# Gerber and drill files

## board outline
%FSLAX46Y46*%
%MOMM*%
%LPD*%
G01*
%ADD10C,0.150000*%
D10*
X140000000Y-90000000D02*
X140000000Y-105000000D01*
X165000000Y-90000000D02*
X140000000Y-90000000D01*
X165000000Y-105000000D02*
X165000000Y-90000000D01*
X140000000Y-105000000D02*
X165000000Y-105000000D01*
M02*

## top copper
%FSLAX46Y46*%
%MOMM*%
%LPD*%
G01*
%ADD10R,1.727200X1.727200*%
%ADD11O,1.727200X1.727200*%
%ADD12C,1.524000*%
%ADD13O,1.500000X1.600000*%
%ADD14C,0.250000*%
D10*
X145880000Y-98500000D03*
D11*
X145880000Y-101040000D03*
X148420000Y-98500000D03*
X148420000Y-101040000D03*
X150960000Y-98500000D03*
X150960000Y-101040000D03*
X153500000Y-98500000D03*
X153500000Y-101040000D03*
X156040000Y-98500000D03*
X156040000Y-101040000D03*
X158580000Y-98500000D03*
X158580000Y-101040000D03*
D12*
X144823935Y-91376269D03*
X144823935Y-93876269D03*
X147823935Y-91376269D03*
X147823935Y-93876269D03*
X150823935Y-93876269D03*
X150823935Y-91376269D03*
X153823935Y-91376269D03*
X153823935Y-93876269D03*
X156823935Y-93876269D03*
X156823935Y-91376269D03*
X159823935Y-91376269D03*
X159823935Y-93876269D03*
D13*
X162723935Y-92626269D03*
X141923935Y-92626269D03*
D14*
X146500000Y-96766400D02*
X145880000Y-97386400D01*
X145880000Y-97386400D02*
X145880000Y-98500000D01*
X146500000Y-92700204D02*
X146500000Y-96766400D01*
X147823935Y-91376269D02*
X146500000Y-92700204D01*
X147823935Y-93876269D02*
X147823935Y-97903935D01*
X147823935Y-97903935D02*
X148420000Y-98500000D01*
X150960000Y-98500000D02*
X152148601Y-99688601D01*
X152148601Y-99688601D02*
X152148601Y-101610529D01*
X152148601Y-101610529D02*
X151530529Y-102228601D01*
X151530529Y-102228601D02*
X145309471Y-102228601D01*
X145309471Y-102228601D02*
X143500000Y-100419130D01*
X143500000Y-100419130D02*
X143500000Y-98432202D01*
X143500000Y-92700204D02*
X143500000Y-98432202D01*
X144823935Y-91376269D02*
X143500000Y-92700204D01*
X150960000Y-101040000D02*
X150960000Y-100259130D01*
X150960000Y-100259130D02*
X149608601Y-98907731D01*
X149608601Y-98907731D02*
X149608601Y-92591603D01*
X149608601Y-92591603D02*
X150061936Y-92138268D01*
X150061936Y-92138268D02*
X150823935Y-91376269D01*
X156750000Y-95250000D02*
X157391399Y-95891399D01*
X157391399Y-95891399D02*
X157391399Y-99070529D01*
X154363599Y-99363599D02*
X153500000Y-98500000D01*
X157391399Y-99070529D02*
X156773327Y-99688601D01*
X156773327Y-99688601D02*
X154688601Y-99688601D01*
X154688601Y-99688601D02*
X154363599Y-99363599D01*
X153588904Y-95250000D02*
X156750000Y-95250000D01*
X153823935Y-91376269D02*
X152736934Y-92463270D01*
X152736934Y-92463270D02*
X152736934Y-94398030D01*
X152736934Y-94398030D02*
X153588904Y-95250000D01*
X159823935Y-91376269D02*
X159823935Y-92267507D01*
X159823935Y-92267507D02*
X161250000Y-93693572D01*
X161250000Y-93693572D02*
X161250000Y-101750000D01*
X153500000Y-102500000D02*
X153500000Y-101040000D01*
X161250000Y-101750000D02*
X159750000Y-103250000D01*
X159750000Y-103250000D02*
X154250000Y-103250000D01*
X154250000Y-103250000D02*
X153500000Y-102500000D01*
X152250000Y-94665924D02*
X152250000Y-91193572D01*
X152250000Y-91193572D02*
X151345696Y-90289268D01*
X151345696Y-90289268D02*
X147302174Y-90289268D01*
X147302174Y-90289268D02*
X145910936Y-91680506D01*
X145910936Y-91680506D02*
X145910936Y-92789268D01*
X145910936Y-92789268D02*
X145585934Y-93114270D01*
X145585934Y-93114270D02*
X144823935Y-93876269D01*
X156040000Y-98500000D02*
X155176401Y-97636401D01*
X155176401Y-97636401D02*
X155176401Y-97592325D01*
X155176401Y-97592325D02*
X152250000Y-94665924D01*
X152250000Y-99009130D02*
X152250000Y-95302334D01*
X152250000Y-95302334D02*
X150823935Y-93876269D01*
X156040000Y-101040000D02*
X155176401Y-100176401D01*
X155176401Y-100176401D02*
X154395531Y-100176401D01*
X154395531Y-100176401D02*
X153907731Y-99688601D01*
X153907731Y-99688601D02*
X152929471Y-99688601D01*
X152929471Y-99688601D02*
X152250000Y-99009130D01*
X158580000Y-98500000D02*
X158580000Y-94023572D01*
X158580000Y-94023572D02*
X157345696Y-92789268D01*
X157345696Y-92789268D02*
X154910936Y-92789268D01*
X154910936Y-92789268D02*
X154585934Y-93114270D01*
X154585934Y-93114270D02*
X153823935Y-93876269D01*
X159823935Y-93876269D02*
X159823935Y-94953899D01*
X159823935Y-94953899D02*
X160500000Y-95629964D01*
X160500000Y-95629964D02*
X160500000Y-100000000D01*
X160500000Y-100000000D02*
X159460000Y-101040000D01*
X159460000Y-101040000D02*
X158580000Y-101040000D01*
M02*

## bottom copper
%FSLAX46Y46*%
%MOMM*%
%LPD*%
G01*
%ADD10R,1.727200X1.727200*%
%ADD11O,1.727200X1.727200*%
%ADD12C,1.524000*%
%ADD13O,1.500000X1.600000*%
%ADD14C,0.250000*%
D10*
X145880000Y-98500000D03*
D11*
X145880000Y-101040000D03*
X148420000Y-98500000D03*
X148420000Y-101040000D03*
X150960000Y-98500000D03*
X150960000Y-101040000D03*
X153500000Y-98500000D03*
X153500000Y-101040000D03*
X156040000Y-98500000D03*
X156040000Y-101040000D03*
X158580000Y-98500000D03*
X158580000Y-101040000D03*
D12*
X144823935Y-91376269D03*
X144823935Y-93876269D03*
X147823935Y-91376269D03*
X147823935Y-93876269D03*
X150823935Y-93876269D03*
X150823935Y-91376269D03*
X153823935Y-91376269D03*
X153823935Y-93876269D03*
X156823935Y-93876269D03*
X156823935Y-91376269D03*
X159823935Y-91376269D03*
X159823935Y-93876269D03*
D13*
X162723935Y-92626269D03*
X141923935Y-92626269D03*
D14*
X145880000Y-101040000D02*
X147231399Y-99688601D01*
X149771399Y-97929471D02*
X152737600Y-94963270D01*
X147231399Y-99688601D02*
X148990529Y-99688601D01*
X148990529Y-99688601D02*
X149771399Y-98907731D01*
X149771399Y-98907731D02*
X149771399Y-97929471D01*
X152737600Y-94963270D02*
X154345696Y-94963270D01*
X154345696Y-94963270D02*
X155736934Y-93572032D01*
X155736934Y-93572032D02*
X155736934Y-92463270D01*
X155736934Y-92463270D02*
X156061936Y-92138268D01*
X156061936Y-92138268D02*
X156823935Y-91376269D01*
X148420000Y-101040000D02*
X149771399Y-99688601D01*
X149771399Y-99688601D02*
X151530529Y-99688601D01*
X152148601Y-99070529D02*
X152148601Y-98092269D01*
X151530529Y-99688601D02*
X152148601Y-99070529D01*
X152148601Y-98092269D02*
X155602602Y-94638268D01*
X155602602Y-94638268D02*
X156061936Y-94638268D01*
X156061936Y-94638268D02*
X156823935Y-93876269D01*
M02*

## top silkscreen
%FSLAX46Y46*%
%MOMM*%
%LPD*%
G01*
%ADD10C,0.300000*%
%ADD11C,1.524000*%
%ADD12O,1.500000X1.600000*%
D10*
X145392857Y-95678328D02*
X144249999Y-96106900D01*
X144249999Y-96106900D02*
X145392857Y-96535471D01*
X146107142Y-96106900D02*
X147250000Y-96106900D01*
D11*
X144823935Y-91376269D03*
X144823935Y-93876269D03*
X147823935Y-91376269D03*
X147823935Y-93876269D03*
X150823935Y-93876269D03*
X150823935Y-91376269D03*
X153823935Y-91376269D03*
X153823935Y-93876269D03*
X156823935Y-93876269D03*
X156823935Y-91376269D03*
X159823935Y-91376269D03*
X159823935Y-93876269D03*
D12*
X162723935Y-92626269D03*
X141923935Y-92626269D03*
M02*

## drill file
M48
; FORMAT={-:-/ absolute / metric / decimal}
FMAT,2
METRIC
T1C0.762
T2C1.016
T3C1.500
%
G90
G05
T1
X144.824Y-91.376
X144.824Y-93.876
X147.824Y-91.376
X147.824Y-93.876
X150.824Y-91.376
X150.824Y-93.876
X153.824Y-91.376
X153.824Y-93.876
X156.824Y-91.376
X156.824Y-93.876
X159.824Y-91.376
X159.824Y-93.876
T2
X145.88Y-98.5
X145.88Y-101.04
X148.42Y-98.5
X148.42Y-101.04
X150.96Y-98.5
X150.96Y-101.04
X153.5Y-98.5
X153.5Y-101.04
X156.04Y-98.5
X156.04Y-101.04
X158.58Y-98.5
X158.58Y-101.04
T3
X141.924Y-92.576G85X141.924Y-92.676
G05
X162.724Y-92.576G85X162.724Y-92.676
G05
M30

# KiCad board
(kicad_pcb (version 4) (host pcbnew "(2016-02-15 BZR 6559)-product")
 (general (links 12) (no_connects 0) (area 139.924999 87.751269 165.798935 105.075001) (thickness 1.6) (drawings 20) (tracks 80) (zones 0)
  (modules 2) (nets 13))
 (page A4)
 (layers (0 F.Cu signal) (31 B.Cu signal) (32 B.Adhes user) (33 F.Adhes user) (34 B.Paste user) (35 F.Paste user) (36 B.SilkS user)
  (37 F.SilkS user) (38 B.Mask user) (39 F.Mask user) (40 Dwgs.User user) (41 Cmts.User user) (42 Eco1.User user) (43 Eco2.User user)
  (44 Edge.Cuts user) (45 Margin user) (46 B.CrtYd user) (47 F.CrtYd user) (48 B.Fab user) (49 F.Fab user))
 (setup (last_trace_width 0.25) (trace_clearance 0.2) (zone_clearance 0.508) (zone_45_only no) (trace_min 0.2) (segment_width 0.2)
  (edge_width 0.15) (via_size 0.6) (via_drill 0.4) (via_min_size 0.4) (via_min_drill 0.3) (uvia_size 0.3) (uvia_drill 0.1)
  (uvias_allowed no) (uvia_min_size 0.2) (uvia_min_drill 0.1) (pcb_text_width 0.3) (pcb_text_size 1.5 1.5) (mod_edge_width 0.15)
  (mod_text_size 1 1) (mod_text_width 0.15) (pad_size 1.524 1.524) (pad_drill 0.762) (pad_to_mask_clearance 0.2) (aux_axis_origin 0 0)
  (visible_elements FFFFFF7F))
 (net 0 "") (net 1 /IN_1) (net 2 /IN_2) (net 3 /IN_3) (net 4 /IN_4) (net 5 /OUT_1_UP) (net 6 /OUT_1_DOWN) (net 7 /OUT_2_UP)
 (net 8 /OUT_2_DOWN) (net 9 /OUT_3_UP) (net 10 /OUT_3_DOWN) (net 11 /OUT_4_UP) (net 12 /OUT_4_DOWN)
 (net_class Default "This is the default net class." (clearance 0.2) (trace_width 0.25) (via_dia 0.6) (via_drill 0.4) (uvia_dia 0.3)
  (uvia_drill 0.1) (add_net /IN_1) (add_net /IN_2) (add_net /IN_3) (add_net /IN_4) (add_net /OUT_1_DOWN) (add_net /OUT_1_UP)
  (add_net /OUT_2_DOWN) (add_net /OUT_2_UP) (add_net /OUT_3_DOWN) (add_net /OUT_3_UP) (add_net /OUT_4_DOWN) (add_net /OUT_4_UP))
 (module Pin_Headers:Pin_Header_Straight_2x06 (layer B.Cu) (at 145.88 98.5 270)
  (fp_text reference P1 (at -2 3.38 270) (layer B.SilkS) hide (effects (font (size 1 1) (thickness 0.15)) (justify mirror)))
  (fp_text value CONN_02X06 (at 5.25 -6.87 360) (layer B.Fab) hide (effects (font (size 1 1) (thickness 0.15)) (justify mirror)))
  (pad 1 thru_hole rect (at 0 0 270) (size 1.7272 1.7272) (drill 1.016) (layers *.Cu *.Mask B.SilkS) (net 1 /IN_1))
  (pad 2 thru_hole oval (at 2.54 0 270) (size 1.7272 1.7272) (drill 1.016) (layers *.Cu *.Mask B.SilkS) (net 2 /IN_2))
  (pad 3 thru_hole oval (at 0 -2.54 270) (size 1.7272 1.7272) (drill 1.016) (layers *.Cu *.Mask B.SilkS) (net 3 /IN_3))
  (pad 4 thru_hole oval (at 2.54 -2.54 270) (size 1.7272 1.7272) (drill 1.016) (layers *.Cu *.Mask B.SilkS) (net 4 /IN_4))
  (pad 5 thru_hole oval (at 0 -5.08 270) (size 1.7272 1.7272) (drill 1.016) (layers *.Cu *.Mask B.SilkS) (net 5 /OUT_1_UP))
  (pad 6 thru_hole oval (at 2.54 -5.08 270) (size 1.7272 1.7272) (drill 1.016) (layers *.Cu *.Mask B.SilkS) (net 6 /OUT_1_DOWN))
  (pad 7 thru_hole oval (at 0 -7.62 270) (size 1.7272 1.7272) (drill 1.016) (layers *.Cu *.Mask B.SilkS) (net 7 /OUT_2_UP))
  (pad 8 thru_hole oval (at 2.54 -7.62 270) (size 1.7272 1.7272) (drill 1.016) (layers *.Cu *.Mask B.SilkS) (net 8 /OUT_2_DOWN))
  (pad 9 thru_hole oval (at 0 -10.16 270) (size 1.7272 1.7272) (drill 1.016) (layers *.Cu *.Mask B.SilkS) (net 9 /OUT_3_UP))
  (pad 10 thru_hole oval (at 2.54 -10.16 270) (size 1.7272 1.7272) (drill 1.016) (layers *.Cu *.Mask B.SilkS) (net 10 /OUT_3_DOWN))
  (pad 11 thru_hole oval (at 0 -12.7 270) (size 1.7272 1.7272) (drill 1.016) (layers *.Cu *.Mask B.SilkS) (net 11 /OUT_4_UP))
  (pad 12 thru_hole oval (at 2.54 -12.7 270) (size 1.7272 1.7272) (drill 1.016) (layers *.Cu *.Mask B.SilkS) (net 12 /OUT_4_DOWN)))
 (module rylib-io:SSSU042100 (layer F.Cu) (at 144.823935 91.376269)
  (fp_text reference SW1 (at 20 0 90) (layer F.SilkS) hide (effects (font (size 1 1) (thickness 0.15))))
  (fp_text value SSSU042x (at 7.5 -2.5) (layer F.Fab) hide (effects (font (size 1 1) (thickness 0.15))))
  (pad 5 thru_hole circle (at 0 0) (size 1.524 1.524) (drill 0.762) (layers *.Cu *.Mask F.SilkS) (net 5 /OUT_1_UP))
  (pad 7 thru_hole circle (at 0 2.5) (size 1.524 1.524) (drill 0.762) (layers *.Cu *.Mask F.SilkS) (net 9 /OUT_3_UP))
  (pad 1 thru_hole circle (at 3 0) (size 1.524 1.524) (drill 0.762) (layers *.Cu *.Mask F.SilkS) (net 1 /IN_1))
  (pad 3 thru_hole circle (at 3 2.5) (size 1.524 1.524) (drill 0.762) (layers *.Cu *.Mask F.SilkS) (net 3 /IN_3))
  (pad 11 thru_hole circle (at 6 2.5) (size 1.524 1.524) (drill 0.762) (layers *.Cu *.Mask F.SilkS) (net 10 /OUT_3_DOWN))
  (pad 9 thru_hole circle (at 6 0) (size 1.524 1.524) (drill 0.762) (layers *.Cu *.Mask F.SilkS) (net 6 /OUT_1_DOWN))
  (pad 6 thru_hole circle (at 9 0) (size 1.524 1.524) (drill 0.762) (layers *.Cu *.Mask F.SilkS) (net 7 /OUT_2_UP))
  (pad 8 thru_hole circle (at 9 2.5) (size 1.524 1.524) (drill 0.762) (layers *.Cu *.Mask F.SilkS) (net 11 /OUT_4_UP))
  (pad 4 thru_hole circle (at 12 2.5) (size 1.524 1.524) (drill 0.762) (layers *.Cu *.Mask F.SilkS) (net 4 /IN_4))
  (pad 2 thru_hole circle (at 12 0) (size 1.524 1.524) (drill 0.762) (layers *.Cu *.Mask F.SilkS) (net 2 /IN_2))
  (pad 10 thru_hole circle (at 15 0) (size 1.524 1.524) (drill 0.762) (layers *.Cu *.Mask F.SilkS) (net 8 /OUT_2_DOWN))
  (pad 12 thru_hole circle (at 15 2.5) (size 1.524 1.524) (drill 0.762) (layers *.Cu *.Mask F.SilkS) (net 12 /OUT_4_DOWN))
  (pad "" thru_hole oval (at 17.9 1.25) (size 1.5 1.6) (drill oval 1.5 1.6) (layers *.Cu *.Mask F.SilkS))
  (pad "" thru_hole oval (at -2.9 1.25) (size 1.5 1.6) (drill oval 1.5 1.6) (layers *.Cu *.Mask F.SilkS)))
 (gr_line (start 140 90) (end 140 105) (layer Edge.Cuts) (width 0.15))
 (gr_line (start 165 90) (end 140 90) (layer Edge.Cuts) (width 0.15))
 (gr_line (start 165 105) (end 165 90) (layer Edge.Cuts) (width 0.15))
 (gr_line (start 140 105) (end 165 105) (layer Edge.Cuts) (width 0.15))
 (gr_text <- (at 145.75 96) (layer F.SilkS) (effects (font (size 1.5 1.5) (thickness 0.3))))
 (segment (start 146.5 96.7664) (end 145.88 97.3864) (width 0.25) (layer F.Cu) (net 1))
 (segment (start 145.88 97.3864) (end 145.88 98.5) (width 0.25) (layer F.Cu) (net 1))
 (segment (start 146.5 92.700204) (end 146.5 96.7664) (width 0.25) (layer F.Cu) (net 1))
 (segment (start 147.823935 91.376269) (end 146.5 92.700204) (width 0.25) (layer F.Cu) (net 1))
 (segment (start 145.88 101.04) (end 147.231399 99.688601) (width 0.25) (layer B.Cu) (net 2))
 (segment (start 149.771399 97.929471) (end 152.7376 94.96327) (width 0.25) (layer B.Cu) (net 2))
 (segment (start 147.231399 99.688601) (end 148.990529 99.688601) (width 0.25) (layer B.Cu) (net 2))
 (segment (start 148.990529 99.688601) (end 149.771399 98.907731) (width 0.25) (layer B.Cu) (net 2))
 (segment (start 149.771399 98.907731) (end 149.771399 97.929471) (width 0.25) (layer B.Cu) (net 2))
 (segment (start 152.7376 94.96327) (end 154.345696 94.96327) (width 0.25) (layer B.Cu) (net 2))
 (segment (start 154.345696 94.96327) (end 155.736934 93.572032) (width 0.25) (layer B.Cu) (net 2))
 (segment (start 155.736934 93.572032) (end 155.736934 92.46327) (width 0.25) (layer B.Cu) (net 2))
 (segment (start 155.736934 92.46327) (end 156.061936 92.138268) (width 0.25) (layer B.Cu) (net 2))
 (segment (start 156.061936 92.138268) (end 156.823935 91.376269) (width 0.25) (layer B.Cu) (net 2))
 (segment (start 147.823935 93.876269) (end 147.823935 97.903935) (width 0.25) (layer F.Cu) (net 3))
 (segment (start 147.823935 97.903935) (end 148.42 98.5) (width 0.25) (layer F.Cu) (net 3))
 (segment (start 148.42 101.04) (end 149.771399 99.688601) (width 0.25) (layer B.Cu) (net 4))
 (segment (start 149.771399 99.688601) (end 151.530529 99.688601) (width 0.25) (layer B.Cu) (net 4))
 (segment (start 152.148601 99.070529) (end 152.148601 98.092269) (width 0.25) (layer B.Cu) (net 4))
 (segment (start 151.530529 99.688601) (end 152.148601 99.070529) (width 0.25) (layer B.Cu) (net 4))
 (segment (start 152.148601 98.092269) (end 155.602602 94.638268) (width 0.25) (layer B.Cu) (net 4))
 (segment (start 155.602602 94.638268) (end 156.061936 94.638268) (width 0.25) (layer B.Cu) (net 4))
 (segment (start 156.061936 94.638268) (end 156.823935 93.876269) (width 0.25) (layer B.Cu) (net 4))
 (segment (start 150.96 98.5) (end 152.148601 99.688601) (width 0.25) (layer F.Cu) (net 5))
 (segment (start 152.148601 99.688601) (end 152.148601 101.610529) (width 0.25) (layer F.Cu) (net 5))
 (segment (start 152.148601 101.610529) (end 151.530529 102.228601) (width 0.25) (layer F.Cu) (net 5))
 (segment (start 151.530529 102.228601) (end 145.309471 102.228601) (width 0.25) (layer F.Cu) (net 5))
 (segment (start 145.309471 102.228601) (end 143.5 100.41913) (width 0.25) (layer F.Cu) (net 5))
 (segment (start 143.5 100.41913) (end 143.5 98.432202) (width 0.25) (layer F.Cu) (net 5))
 (segment (start 143.5 92.700204) (end 143.5 98.432202) (width 0.25) (layer F.Cu) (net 5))
 (segment (start 144.823935 91.376269) (end 143.5 92.700204) (width 0.25) (layer F.Cu) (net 5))
 (segment (start 150.96 101.04) (end 150.96 100.25913) (width 0.25) (layer F.Cu) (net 6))
 (segment (start 150.96 100.25913) (end 149.608601 98.907731) (width 0.25) (layer F.Cu) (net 6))
 (segment (start 149.608601 98.907731) (end 149.608601 92.591603) (width 0.25) (layer F.Cu) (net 6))
 (segment (start 149.608601 92.591603) (end 150.061936 92.138268) (width 0.25) (layer F.Cu) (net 6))
 (segment (start 150.061936 92.138268) (end 150.823935 91.376269) (width 0.25) (layer F.Cu) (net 6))
 (segment (start 156.75 95.25) (end 157.391399 95.891399) (width 0.25) (layer F.Cu) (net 7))
 (segment (start 157.391399 95.891399) (end 157.391399 99.070529) (width 0.25) (layer F.Cu) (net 7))
 (segment (start 154.363599 99.363599) (end 153.5 98.5) (width 0.25) (layer F.Cu) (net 7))
 (segment (start 157.391399 99.070529) (end 156.773327 99.688601) (width 0.25) (layer F.Cu) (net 7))
 (segment (start 156.773327 99.688601) (end 154.688601 99.688601) (width 0.25) (layer F.Cu) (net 7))
 (segment (start 154.688601 99.688601) (end 154.363599 99.363599) (width 0.25) (layer F.Cu) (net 7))
 (segment (start 153.588904 95.25) (end 156.75 95.25) (width 0.25) (layer F.Cu) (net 7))
 (segment (start 153.823935 91.376269) (end 152.736934 92.46327) (width 0.25) (layer F.Cu) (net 7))
 (segment (start 152.736934 92.46327) (end 152.736934 94.39803) (width 0.25) (layer F.Cu) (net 7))
 (segment (start 152.736934 94.39803) (end 153.588904 95.25) (width 0.25) (layer F.Cu) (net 7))
 (segment (start 159.823935 91.376269) (end 159.823935 92.267507) (width 0.25) (layer F.Cu) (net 8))
 (segment (start 159.823935 92.267507) (end 161.25 93.693572) (width 0.25) (layer F.Cu) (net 8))
 (segment (start 161.25 93.693572) (end 161.25 101.75) (width 0.25) (layer F.Cu) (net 8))
 (segment (start 153.5 102.5) (end 153.5 101.04) (width 0.25) (layer F.Cu) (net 8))
 (segment (start 161.25 101.75) (end 159.75 103.25) (width 0.25) (layer F.Cu) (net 8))
 (segment (start 159.75 103.25) (end 154.25 103.25) (width 0.25) (layer F.Cu) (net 8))
 (segment (start 154.25 103.25) (end 153.5 102.5) (width 0.25) (layer F.Cu) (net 8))
 (segment (start 152.25 94.665924) (end 152.25 91.193572) (width 0.25) (layer F.Cu) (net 9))
 (segment (start 152.25 91.193572) (end 151.345696 90.289268) (width 0.25) (layer F.Cu) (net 9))
 (segment (start 151.345696 90.289268) (end 147.302174 90.289268) (width 0.25) (layer F.Cu) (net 9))
 (segment (start 147.302174 90.289268) (end 145.910936 91.680506) (width 0.25) (layer F.Cu) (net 9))
 (segment (start 145.910936 91.680506) (end 145.910936 92.789268) (width 0.25) (layer F.Cu) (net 9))
 (segment (start 145.910936 92.789268) (end 145.585934 93.11427) (width 0.25) (layer F.Cu) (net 9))
 (segment (start 145.585934 93.11427) (end 144.823935 93.876269) (width 0.25) (layer F.Cu) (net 9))
 (segment (start 156.04 98.5) (end 155.176401 97.636401) (width 0.25) (layer F.Cu) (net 9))
 (segment (start 155.176401 97.636401) (end 155.176401 97.592325) (width 0.25) (layer F.Cu) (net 9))
 (segment (start 155.176401 97.592325) (end 152.25 94.665924) (width 0.25) (layer F.Cu) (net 9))
 (segment (start 152.25 99.00913) (end 152.25 95.302334) (width 0.25) (layer F.Cu) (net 10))
 (segment (start 152.25 95.302334) (end 150.823935 93.876269) (width 0.25) (layer F.Cu) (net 10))
 (segment (start 156.04 101.04) (end 155.176401 100.176401) (width 0.25) (layer F.Cu) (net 10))
 (segment (start 155.176401 100.176401) (end 154.395531 100.176401) (width 0.25) (layer F.Cu) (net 10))
 (segment (start 154.395531 100.176401) (end 153.907731 99.688601) (width 0.25) (layer F.Cu) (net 10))
 (segment (start 153.907731 99.688601) (end 152.929471 99.688601) (width 0.25) (layer F.Cu) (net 10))
 (segment (start 152.929471 99.688601) (end 152.25 99.00913) (width 0.25) (layer F.Cu) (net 10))
 (segment (start 158.58 98.5) (end 158.58 94.023572) (width 0.25) (layer F.Cu) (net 11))
 (segment (start 158.58 94.023572) (end 157.345696 92.789268) (width 0.25) (layer F.Cu) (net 11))
 (segment (start 157.345696 92.789268) (end 154.910936 92.789268) (width 0.25) (layer F.Cu) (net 11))
 (segment (start 154.910936 92.789268) (end 154.585934 93.11427) (width 0.25) (layer F.Cu) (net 11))
 (segment (start 154.585934 93.11427) (end 153.823935 93.876269) (width 0.25) (layer F.Cu) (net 11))
 (segment (start 159.823935 93.876269) (end 159.823935 94.953899) (width 0.25) (layer F.Cu) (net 12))
 (segment (start 159.823935 94.953899) (end 160.5 95.629964) (width 0.25) (layer F.Cu) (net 12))
 (segment (start 160.5 95.629964) (end 160.5 100) (width 0.25) (layer F.Cu) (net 12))
 (segment (start 160.5 100) (end 159.46 101.04) (width 0.25) (layer F.Cu) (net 12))
 (segment (start 159.46 101.04) (end 158.58 101.04) (width 0.25) (layer F.Cu) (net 12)))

